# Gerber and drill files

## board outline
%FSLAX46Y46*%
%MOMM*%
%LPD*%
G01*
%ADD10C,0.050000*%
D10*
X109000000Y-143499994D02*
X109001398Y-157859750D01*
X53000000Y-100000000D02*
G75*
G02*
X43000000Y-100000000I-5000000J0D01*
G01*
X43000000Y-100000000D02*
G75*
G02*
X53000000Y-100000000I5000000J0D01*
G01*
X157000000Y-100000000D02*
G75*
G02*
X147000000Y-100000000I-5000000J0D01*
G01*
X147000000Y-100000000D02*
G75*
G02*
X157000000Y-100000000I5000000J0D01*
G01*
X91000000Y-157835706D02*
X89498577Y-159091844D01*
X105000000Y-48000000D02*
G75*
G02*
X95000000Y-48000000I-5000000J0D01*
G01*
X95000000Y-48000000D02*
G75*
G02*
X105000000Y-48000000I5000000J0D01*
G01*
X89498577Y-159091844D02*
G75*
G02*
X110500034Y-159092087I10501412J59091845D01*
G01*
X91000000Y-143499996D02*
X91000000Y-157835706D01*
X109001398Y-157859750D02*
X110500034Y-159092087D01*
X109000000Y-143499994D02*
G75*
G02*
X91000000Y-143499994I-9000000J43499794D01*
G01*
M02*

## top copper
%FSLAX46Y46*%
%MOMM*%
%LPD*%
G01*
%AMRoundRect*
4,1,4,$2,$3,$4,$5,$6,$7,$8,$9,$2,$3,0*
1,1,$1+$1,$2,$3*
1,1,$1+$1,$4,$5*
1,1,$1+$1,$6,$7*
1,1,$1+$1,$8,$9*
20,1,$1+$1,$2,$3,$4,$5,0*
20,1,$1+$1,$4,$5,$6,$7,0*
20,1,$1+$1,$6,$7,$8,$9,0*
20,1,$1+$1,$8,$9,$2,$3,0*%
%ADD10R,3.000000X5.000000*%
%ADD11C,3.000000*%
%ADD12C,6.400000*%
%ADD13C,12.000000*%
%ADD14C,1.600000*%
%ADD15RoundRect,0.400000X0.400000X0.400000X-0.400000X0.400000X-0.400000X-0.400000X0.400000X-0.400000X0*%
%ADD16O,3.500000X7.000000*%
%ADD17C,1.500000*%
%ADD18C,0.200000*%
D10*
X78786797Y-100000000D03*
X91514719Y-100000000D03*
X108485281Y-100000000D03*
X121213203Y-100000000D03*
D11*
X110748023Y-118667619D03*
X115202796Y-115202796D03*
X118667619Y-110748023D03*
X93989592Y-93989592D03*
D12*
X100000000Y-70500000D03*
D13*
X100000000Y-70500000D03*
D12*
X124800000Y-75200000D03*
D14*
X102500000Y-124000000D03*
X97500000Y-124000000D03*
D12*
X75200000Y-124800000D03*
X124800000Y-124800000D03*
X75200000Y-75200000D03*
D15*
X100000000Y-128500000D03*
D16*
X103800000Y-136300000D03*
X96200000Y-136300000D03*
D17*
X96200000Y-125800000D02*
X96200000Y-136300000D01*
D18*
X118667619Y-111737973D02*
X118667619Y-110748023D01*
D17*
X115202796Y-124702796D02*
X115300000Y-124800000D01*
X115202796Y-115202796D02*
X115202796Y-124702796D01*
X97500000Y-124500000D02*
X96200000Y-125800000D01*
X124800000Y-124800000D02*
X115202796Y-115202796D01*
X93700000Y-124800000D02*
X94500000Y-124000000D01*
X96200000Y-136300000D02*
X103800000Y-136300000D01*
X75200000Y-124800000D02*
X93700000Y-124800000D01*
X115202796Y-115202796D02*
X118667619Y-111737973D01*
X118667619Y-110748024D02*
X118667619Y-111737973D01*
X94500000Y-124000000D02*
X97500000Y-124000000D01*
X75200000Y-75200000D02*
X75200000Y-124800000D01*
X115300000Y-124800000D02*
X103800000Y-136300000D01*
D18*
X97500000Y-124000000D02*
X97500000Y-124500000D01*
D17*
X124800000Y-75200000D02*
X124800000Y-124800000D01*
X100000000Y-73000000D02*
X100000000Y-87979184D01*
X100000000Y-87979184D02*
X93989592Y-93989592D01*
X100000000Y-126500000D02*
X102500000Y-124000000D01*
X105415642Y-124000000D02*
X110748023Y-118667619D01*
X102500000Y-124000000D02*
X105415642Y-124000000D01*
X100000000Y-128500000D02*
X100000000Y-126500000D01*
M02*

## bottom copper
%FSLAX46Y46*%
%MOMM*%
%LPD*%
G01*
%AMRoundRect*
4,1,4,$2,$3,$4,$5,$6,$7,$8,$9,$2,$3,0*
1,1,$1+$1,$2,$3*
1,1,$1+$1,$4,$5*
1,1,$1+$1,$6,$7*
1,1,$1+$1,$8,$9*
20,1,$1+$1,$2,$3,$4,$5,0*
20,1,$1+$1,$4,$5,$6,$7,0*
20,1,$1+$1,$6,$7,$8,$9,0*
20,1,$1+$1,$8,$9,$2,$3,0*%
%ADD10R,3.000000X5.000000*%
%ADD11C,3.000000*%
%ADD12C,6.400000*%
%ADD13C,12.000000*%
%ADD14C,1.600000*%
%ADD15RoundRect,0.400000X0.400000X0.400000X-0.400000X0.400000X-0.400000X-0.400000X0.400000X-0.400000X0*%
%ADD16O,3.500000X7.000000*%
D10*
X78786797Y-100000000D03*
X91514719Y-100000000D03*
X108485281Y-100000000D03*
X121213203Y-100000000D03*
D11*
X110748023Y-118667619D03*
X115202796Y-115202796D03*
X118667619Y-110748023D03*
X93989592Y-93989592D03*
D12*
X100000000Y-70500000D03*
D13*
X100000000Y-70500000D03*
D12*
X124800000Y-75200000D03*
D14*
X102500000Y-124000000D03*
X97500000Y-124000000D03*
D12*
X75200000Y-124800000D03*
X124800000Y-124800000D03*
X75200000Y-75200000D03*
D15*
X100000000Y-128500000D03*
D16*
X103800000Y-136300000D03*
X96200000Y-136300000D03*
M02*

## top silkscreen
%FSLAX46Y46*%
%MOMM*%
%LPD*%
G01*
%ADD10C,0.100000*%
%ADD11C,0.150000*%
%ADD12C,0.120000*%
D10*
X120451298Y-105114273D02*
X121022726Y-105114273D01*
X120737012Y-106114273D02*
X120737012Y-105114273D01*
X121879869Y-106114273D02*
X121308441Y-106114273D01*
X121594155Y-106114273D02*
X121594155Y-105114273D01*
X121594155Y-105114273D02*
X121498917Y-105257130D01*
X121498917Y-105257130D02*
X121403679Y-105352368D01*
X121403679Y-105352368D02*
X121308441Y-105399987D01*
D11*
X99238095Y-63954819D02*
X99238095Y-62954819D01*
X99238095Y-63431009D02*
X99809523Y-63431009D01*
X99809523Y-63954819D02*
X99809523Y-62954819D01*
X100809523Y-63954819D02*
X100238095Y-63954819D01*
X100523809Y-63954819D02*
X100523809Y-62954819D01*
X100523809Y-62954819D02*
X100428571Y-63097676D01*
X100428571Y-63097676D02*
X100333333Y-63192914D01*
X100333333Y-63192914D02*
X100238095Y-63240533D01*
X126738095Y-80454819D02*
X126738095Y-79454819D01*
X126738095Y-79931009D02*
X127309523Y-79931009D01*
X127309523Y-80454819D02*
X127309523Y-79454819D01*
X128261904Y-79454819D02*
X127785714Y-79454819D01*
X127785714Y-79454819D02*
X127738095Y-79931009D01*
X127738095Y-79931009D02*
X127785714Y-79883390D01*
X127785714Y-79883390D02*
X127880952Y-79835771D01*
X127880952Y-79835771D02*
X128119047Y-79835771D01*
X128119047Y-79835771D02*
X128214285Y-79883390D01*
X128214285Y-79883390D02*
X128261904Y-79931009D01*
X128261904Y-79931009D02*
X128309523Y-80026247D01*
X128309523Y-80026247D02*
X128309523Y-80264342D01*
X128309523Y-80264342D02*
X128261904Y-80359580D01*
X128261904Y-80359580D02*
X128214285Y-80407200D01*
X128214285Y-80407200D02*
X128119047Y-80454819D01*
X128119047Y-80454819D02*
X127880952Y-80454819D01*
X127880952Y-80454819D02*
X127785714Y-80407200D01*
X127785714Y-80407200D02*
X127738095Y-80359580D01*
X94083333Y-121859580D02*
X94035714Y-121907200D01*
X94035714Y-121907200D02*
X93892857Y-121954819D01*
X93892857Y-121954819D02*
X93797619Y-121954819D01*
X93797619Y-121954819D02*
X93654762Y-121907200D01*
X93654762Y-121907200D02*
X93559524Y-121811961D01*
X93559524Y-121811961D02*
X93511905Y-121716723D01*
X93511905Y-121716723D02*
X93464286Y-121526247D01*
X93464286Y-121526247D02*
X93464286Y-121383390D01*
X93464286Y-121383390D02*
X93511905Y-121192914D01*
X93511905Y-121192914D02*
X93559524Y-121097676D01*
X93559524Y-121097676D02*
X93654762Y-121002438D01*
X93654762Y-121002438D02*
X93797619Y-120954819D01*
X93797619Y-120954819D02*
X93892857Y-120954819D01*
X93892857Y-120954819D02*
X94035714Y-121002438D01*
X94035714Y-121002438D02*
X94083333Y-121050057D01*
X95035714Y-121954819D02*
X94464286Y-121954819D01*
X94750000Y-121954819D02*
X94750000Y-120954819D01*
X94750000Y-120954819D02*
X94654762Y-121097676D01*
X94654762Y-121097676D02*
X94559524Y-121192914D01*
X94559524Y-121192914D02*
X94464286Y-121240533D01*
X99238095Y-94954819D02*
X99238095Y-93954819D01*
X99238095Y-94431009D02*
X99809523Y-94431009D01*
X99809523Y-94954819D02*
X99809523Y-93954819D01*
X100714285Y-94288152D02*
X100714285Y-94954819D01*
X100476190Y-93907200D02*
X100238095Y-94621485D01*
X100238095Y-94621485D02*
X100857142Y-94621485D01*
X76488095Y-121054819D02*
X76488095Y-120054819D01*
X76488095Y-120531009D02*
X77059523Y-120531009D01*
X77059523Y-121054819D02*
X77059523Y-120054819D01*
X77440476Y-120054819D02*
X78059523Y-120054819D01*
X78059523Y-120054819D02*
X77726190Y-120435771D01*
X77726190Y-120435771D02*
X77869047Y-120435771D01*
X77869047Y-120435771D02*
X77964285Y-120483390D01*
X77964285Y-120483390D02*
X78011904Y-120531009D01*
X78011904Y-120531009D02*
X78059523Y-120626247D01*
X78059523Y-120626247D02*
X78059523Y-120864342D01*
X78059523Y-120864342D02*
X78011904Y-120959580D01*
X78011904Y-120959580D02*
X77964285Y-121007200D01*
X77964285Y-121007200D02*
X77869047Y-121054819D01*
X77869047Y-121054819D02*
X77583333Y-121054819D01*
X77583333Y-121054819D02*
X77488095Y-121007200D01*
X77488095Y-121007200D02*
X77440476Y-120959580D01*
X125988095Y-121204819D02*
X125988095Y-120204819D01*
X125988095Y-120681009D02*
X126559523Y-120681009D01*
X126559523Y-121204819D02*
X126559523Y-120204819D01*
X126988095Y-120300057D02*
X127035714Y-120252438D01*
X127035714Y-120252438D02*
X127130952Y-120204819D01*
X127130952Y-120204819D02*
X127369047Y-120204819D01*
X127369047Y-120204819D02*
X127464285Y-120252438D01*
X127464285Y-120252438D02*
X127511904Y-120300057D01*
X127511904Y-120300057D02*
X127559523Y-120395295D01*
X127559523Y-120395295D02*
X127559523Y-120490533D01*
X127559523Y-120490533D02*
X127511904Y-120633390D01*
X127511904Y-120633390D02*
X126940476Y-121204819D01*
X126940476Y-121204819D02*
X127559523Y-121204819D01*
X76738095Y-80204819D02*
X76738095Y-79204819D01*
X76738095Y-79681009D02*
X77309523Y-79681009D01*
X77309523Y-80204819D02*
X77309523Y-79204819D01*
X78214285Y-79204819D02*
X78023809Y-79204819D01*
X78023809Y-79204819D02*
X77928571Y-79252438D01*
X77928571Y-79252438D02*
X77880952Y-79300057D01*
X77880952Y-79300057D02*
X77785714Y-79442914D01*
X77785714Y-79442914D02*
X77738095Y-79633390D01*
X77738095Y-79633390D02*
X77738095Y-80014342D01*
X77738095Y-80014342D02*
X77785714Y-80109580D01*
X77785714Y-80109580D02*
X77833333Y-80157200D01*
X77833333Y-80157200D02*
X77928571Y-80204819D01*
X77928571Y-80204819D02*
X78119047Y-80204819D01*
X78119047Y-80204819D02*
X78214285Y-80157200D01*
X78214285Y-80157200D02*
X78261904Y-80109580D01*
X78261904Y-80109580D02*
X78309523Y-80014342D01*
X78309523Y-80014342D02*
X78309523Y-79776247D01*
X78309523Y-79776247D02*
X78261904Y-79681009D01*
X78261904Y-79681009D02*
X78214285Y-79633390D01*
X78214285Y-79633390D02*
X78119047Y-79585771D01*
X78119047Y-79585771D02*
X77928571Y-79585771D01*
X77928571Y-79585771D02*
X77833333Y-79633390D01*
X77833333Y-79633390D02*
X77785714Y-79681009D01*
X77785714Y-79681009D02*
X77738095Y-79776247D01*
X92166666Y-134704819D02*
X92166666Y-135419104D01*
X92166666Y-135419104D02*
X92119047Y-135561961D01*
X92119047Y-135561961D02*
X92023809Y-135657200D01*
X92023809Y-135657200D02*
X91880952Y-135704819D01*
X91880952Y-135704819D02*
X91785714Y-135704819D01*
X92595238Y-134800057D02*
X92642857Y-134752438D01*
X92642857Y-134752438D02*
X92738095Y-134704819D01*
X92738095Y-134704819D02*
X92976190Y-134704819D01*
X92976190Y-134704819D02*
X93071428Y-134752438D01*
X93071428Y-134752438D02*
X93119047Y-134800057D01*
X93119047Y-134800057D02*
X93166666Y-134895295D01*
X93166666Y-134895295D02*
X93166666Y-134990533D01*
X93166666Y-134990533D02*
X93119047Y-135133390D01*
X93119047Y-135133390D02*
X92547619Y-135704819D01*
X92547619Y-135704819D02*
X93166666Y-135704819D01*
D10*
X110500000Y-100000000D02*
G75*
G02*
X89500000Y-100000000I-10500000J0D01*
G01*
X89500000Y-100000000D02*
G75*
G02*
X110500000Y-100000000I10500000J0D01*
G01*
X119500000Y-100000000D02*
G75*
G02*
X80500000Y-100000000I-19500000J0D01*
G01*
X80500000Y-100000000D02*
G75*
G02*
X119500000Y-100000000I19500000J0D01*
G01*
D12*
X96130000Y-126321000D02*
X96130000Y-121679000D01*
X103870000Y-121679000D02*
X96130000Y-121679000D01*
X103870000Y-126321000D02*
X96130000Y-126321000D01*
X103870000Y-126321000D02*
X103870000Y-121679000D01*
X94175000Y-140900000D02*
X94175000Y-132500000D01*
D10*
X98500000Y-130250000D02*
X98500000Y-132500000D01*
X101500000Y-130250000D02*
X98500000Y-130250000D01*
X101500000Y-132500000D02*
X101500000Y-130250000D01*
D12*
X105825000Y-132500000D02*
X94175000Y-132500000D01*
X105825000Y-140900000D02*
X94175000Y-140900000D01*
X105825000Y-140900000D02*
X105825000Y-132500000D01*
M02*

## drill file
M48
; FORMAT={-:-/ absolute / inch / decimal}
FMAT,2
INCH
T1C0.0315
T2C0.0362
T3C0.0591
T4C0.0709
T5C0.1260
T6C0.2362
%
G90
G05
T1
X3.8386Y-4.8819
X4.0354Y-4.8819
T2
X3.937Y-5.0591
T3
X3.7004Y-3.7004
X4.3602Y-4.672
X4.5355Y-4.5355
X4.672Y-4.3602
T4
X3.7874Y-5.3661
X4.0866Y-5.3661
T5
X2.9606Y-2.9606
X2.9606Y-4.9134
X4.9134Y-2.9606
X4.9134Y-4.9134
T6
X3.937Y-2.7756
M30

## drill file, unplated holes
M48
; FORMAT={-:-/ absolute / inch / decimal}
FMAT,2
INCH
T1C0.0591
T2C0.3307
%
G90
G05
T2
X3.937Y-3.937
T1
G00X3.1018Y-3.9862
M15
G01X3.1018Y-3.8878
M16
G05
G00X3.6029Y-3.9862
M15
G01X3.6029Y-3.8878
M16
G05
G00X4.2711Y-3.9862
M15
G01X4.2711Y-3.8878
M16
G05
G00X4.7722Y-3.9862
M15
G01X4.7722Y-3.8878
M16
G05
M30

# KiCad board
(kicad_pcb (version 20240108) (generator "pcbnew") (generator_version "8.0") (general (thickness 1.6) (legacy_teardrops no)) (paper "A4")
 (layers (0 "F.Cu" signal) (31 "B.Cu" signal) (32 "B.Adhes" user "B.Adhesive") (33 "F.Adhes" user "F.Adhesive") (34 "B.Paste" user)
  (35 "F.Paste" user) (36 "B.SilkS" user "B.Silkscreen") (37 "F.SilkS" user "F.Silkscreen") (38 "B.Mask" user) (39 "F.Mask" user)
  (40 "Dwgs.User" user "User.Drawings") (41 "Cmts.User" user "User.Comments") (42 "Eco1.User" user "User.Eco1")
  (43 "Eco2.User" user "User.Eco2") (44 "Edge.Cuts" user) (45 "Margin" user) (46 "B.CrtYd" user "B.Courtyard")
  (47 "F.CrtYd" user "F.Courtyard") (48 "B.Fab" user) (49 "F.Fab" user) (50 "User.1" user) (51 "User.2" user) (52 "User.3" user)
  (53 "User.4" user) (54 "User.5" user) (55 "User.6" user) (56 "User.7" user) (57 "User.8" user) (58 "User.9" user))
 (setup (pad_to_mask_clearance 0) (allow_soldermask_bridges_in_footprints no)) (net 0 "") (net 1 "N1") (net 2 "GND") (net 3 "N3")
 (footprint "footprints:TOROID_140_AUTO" (layer "F.Cu") (at 100 100 45)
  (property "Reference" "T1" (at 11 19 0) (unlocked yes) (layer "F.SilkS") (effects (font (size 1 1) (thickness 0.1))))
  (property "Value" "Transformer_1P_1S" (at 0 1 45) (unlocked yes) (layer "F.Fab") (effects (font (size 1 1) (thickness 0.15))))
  (fp_circle (center 0 0) (end 10.5 0) (stroke (width 0.1) (type default)) (fill none) (layer "F.SilkS"))
  (fp_circle (center 0 0) (end 19.5 0) (stroke (width 0.1) (type default)) (fill none) (layer "F.SilkS"))
  (pad "" np_thru_hole rect (at -15 -15 90) (size 5 3) (drill oval 4 1.5) (layers "F&B.Cu"))
  (pad "" np_thru_hole rect (at -6 -6 90) (size 5 3) (drill oval 4 1.5) (layers "F&B.Cu"))
  (pad "" np_thru_hole rect (at 6 6 90) (size 5 3) (drill oval 4 1.5) (layers "F&B.Cu"))
  (pad "" np_thru_hole rect (at 15 15 90) (size 5 3) (drill oval 4 1.5) (layers "F&B.Cu"))
  (pad "1" thru_hole circle (at -5.6 20.8 45) (size 3 3) (drill 1.5) (layers "*.Cu" "*.Mask") (remove_unused_layers no) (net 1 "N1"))
  (pad "2" thru_hole circle (at 0 21.5 45) (size 3 3) (drill 1.5) (layers "*.Cu" "*.Mask") (remove_unused_layers no) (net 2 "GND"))
  (pad "3" thru_hole circle (at 5.6 20.8 45) (size 3 3) (drill 1.5) (layers "*.Cu" "*.Mask") (remove_unused_layers no) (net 2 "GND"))
  (pad "4" thru_hole circle (at 0 -8.500001 45) (size 3 3) (drill 1.5) (layers "*.Cu" "*.Mask") (remove_unused_layers no) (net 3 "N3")))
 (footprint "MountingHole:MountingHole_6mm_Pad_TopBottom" (layer "F.Cu") (at 100 70.5)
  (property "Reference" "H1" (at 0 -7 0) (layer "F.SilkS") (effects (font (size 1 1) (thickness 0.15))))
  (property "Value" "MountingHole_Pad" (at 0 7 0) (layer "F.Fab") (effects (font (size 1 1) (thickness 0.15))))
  (pad "1" thru_hole circle (at 0 0) (size 6.4 6.4) (drill 6) (layers "*.Cu" "*.Mask") (remove_unused_layers no) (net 3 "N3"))
  (pad "1" connect circle (at 0 0) (size 12 12) (layers "F.Cu" "F.Mask") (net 3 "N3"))
  (pad "1" connect circle (at 0 0) (size 12 12) (layers "B.Cu" "B.Mask") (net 3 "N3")))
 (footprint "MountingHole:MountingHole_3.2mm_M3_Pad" (layer "F.Cu") (at 124.8 75.2)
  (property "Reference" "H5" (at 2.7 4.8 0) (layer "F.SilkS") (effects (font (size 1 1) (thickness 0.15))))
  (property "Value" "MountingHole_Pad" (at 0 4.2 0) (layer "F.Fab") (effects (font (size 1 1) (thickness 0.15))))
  (pad "1" thru_hole circle (at 0 0) (size 6.4 6.4) (drill 3.2) (layers "*.Cu" "*.Mask") (remove_unused_layers no) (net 2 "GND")))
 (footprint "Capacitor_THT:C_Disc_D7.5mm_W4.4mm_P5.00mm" (layer "F.Cu") (at 102.5 124 180)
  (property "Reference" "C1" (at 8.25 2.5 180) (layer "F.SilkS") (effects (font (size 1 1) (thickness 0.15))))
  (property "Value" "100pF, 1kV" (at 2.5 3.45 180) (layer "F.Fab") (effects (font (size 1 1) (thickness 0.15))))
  (fp_line (start 6.37 -2.321) (end 6.37 2.321) (stroke (width 0.12) (type solid)) (layer "F.SilkS"))
  (fp_line (start -1.37 2.321) (end 6.37 2.321) (stroke (width 0.12) (type solid)) (layer "F.SilkS"))
  (fp_line (start -1.37 -2.321) (end 6.37 -2.321) (stroke (width 0.12) (type solid)) (layer "F.SilkS"))
  (fp_line (start -1.37 -2.321) (end -1.37 2.321) (stroke (width 0.12) (type solid)) (layer "F.SilkS"))
  (pad "1" thru_hole circle (at 0 0 180) (size 1.6 1.6) (drill 0.8) (layers "*.Cu" "*.Mask") (remove_unused_layers no) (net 1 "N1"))
  (pad "2" thru_hole circle (at 5 0 180) (size 1.6 1.6) (drill 0.8) (layers "*.Cu" "*.Mask") (remove_unused_layers no) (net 2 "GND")))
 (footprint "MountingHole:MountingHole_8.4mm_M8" (layer "F.Cu") (at 100 100)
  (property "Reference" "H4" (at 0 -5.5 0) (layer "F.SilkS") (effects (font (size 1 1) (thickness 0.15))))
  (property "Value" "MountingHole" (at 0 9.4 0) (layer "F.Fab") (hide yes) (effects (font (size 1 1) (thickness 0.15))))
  (pad "" np_thru_hole circle (at 0 0) (size 8.4 8.4) (drill 8.4) (layers "*.Cu" "*.Mask")))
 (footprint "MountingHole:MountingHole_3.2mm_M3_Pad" (layer "F.Cu") (at 75.2 124.8)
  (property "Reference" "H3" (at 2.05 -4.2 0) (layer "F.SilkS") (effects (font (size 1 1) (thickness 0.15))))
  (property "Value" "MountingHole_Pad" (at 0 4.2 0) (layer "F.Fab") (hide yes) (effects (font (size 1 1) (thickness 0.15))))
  (pad "1" thru_hole circle (at 0 0) (size 6.4 6.4) (drill 3.2) (layers "*.Cu" "*.Mask") (remove_unused_layers no) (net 2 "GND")))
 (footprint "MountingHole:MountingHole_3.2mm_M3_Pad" (layer "F.Cu") (at 124.8 124.8)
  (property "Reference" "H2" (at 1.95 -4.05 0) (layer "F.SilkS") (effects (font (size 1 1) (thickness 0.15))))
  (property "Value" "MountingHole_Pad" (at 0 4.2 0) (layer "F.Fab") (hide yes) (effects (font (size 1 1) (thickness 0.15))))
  (pad "1" thru_hole circle (at 0 0) (size 6.4 6.4) (drill 3.2) (layers "*.Cu" "*.Mask") (remove_unused_layers no) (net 2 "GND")))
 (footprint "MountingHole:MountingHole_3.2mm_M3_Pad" (layer "F.Cu") (at 75.2 75.2)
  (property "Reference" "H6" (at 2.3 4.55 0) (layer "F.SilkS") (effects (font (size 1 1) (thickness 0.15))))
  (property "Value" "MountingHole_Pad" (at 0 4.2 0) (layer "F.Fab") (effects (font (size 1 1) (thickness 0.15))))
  (pad "1" thru_hole circle (at 0 0) (size 6.4 6.4) (drill 3.2) (layers "*.Cu" "*.Mask") (remove_unused_layers no) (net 2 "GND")))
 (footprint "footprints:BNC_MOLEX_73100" (layer "F.Cu") (at 100 128.5 180)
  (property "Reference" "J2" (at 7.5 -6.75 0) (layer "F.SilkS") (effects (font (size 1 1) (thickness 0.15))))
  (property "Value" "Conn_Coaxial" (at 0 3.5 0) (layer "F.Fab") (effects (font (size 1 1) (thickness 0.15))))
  (fp_line (start 5.825 -12.4) (end 5.825 -4) (stroke (width 0.12) (type solid)) (layer "F.SilkS"))
  (fp_line (start 1.5 -1.75) (end 1.5 -4) (stroke (width 0.1) (type default)) (layer "F.SilkS"))
  (fp_line (start -1.5 -1.75) (end 1.5 -1.75) (stroke (width 0.1) (type default)) (layer "F.SilkS"))
  (fp_line (start -1.5 -4) (end -1.5 -1.75) (stroke (width 0.1) (type default)) (layer "F.SilkS"))
  (fp_line (start -5.825 -4) (end 5.825 -4) (stroke (width 0.12) (type solid)) (layer "F.SilkS"))
  (fp_line (start -5.825 -12.4) (end 5.825 -12.4) (stroke (width 0.12) (type solid)) (layer "F.SilkS"))
  (fp_line (start -5.825 -12.4) (end -5.825 -4) (stroke (width 0.12) (type solid)) (layer "F.SilkS"))
  (pad "1" thru_hole roundrect (at 0 0 180) (size 1.6 1.6) (drill 0.92) (layers "*.Cu" "*.Mask") (remove_unused_layers no)
   (roundrect_rratio 0.25) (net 1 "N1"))
  (pad "2" thru_hole oval (at -3.8 -7.8 180) (size 3.5 7) (drill 1.8) (layers "*.Cu" "*.Mask") (remove_unused_layers no) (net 2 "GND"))
  (pad "2" thru_hole oval (at 3.8 -7.8 180) (size 3.5 7) (drill 1.8) (layers "*.Cu" "*.Mask") (remove_unused_layers no) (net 2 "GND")))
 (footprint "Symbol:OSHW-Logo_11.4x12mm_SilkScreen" (layer "B.Cu") (at 65 110.5 180)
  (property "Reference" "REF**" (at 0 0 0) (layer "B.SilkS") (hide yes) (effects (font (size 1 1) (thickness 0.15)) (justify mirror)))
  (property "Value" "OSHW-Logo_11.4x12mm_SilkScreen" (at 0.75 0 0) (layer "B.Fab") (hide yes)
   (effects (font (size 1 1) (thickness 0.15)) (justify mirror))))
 (gr_line (start 109 143.499994) (end 109.001398 157.85975) (stroke (width 0.05) (type default)) (layer "Edge.Cuts"))
 (gr_circle (center 48 100) (end 53 100) (stroke (width 0.05) (type default)) (fill none) (layer "Edge.Cuts"))
 (gr_circle (center 152 100) (end 157 100) (stroke (width 0.05) (type default)) (fill none) (layer "Edge.Cuts"))
 (gr_line (start 91 157.835706) (end 89.498577 159.091844) (stroke (width 0.05) (type default)) (layer "Edge.Cuts"))
 (gr_circle (center 100 48) (end 105 48) (stroke (width 0.05) (type default)) (fill none) (layer "Edge.Cuts"))
 (gr_arc (start 89.498577 159.091844) (mid 100.000087 39.982287) (end 110.500034 159.092087) (stroke (width 0.05) (type default))
  (layer "Edge.Cuts"))
 (gr_line (start 91 143.499996) (end 91 157.835706) (stroke (width 0.05) (type default)) (layer "Edge.Cuts"))
 (gr_line (start 109.001398 157.85975) (end 110.500034 159.092087) (stroke (width 0.05) (type default)) (layer "Edge.Cuts"))
 (gr_arc (start 109 143.499994) (mid 100 144.421278) (end 91 143.499996) (stroke (width 0.05) (type default)) (layer "Edge.Cuts"))
 (segment (start 96.2 125.8) (end 96.2 136.3) (width 1.5) (layer "F.Cu") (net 2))
 (segment (start 118.667619 111.737973) (end 118.667619 110.748023) (width 0.2) (layer "F.Cu") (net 2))
 (segment (start 115.202796 124.702796) (end 115.3 124.8) (width 1.5) (layer "F.Cu") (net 2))
 (segment (start 115.202796 115.202796) (end 115.202796 124.702796) (width 1.5) (layer "F.Cu") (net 2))
 (segment (start 97.5 124.5) (end 96.2 125.8) (width 1.5) (layer "F.Cu") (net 2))
 (segment (start 124.8 124.8) (end 115.202796 115.202796) (width 1.5) (layer "F.Cu") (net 2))
 (segment (start 93.7 124.8) (end 94.5 124) (width 1.5) (layer "F.Cu") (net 2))
 (segment (start 96.2 136.3) (end 103.8 136.3) (width 1.5) (layer "F.Cu") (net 2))
 (segment (start 75.2 124.8) (end 93.7 124.8) (width 1.5) (layer "F.Cu") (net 2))
 (segment (start 115.202796 115.202796) (end 118.667619 111.737973) (width 1.5) (layer "F.Cu") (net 2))
 (segment (start 118.667619 110.748024) (end 118.667619 111.737973) (width 1.5) (layer "F.Cu") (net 2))
 (segment (start 94.5 124) (end 97.5 124) (width 1.5) (layer "F.Cu") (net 2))
 (segment (start 75.2 75.2) (end 75.2 124.8) (width 1.5) (layer "F.Cu") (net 2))
 (segment (start 115.3 124.8) (end 103.8 136.3) (width 1.5) (layer "F.Cu") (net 2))
 (segment (start 97.5 124) (end 97.5 124.5) (width 0.2) (layer "F.Cu") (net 2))
 (segment (start 124.8 75.2) (end 124.8 124.8) (width 1.5) (layer "F.Cu") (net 2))
 (segment (start 100 73) (end 100 87.979184) (width 1.5) (layer "F.Cu") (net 3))
 (segment (start 100 87.979184) (end 93.989592 93.989592) (width 1.5) (layer "F.Cu") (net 3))
 (segment (start 100 126.5) (end 102.5 124) (width 1.5) (layer "F.Cu") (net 1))
 (segment (start 105.415642 124) (end 110.748023 118.667619) (width 1.5) (layer "F.Cu") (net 1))
 (segment (start 102.5 124) (end 105.415642 124) (width 1.5) (layer "F.Cu") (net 1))
 (segment (start 100 128.5) (end 100 126.5) (width 1.5) (layer "F.Cu") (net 1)))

